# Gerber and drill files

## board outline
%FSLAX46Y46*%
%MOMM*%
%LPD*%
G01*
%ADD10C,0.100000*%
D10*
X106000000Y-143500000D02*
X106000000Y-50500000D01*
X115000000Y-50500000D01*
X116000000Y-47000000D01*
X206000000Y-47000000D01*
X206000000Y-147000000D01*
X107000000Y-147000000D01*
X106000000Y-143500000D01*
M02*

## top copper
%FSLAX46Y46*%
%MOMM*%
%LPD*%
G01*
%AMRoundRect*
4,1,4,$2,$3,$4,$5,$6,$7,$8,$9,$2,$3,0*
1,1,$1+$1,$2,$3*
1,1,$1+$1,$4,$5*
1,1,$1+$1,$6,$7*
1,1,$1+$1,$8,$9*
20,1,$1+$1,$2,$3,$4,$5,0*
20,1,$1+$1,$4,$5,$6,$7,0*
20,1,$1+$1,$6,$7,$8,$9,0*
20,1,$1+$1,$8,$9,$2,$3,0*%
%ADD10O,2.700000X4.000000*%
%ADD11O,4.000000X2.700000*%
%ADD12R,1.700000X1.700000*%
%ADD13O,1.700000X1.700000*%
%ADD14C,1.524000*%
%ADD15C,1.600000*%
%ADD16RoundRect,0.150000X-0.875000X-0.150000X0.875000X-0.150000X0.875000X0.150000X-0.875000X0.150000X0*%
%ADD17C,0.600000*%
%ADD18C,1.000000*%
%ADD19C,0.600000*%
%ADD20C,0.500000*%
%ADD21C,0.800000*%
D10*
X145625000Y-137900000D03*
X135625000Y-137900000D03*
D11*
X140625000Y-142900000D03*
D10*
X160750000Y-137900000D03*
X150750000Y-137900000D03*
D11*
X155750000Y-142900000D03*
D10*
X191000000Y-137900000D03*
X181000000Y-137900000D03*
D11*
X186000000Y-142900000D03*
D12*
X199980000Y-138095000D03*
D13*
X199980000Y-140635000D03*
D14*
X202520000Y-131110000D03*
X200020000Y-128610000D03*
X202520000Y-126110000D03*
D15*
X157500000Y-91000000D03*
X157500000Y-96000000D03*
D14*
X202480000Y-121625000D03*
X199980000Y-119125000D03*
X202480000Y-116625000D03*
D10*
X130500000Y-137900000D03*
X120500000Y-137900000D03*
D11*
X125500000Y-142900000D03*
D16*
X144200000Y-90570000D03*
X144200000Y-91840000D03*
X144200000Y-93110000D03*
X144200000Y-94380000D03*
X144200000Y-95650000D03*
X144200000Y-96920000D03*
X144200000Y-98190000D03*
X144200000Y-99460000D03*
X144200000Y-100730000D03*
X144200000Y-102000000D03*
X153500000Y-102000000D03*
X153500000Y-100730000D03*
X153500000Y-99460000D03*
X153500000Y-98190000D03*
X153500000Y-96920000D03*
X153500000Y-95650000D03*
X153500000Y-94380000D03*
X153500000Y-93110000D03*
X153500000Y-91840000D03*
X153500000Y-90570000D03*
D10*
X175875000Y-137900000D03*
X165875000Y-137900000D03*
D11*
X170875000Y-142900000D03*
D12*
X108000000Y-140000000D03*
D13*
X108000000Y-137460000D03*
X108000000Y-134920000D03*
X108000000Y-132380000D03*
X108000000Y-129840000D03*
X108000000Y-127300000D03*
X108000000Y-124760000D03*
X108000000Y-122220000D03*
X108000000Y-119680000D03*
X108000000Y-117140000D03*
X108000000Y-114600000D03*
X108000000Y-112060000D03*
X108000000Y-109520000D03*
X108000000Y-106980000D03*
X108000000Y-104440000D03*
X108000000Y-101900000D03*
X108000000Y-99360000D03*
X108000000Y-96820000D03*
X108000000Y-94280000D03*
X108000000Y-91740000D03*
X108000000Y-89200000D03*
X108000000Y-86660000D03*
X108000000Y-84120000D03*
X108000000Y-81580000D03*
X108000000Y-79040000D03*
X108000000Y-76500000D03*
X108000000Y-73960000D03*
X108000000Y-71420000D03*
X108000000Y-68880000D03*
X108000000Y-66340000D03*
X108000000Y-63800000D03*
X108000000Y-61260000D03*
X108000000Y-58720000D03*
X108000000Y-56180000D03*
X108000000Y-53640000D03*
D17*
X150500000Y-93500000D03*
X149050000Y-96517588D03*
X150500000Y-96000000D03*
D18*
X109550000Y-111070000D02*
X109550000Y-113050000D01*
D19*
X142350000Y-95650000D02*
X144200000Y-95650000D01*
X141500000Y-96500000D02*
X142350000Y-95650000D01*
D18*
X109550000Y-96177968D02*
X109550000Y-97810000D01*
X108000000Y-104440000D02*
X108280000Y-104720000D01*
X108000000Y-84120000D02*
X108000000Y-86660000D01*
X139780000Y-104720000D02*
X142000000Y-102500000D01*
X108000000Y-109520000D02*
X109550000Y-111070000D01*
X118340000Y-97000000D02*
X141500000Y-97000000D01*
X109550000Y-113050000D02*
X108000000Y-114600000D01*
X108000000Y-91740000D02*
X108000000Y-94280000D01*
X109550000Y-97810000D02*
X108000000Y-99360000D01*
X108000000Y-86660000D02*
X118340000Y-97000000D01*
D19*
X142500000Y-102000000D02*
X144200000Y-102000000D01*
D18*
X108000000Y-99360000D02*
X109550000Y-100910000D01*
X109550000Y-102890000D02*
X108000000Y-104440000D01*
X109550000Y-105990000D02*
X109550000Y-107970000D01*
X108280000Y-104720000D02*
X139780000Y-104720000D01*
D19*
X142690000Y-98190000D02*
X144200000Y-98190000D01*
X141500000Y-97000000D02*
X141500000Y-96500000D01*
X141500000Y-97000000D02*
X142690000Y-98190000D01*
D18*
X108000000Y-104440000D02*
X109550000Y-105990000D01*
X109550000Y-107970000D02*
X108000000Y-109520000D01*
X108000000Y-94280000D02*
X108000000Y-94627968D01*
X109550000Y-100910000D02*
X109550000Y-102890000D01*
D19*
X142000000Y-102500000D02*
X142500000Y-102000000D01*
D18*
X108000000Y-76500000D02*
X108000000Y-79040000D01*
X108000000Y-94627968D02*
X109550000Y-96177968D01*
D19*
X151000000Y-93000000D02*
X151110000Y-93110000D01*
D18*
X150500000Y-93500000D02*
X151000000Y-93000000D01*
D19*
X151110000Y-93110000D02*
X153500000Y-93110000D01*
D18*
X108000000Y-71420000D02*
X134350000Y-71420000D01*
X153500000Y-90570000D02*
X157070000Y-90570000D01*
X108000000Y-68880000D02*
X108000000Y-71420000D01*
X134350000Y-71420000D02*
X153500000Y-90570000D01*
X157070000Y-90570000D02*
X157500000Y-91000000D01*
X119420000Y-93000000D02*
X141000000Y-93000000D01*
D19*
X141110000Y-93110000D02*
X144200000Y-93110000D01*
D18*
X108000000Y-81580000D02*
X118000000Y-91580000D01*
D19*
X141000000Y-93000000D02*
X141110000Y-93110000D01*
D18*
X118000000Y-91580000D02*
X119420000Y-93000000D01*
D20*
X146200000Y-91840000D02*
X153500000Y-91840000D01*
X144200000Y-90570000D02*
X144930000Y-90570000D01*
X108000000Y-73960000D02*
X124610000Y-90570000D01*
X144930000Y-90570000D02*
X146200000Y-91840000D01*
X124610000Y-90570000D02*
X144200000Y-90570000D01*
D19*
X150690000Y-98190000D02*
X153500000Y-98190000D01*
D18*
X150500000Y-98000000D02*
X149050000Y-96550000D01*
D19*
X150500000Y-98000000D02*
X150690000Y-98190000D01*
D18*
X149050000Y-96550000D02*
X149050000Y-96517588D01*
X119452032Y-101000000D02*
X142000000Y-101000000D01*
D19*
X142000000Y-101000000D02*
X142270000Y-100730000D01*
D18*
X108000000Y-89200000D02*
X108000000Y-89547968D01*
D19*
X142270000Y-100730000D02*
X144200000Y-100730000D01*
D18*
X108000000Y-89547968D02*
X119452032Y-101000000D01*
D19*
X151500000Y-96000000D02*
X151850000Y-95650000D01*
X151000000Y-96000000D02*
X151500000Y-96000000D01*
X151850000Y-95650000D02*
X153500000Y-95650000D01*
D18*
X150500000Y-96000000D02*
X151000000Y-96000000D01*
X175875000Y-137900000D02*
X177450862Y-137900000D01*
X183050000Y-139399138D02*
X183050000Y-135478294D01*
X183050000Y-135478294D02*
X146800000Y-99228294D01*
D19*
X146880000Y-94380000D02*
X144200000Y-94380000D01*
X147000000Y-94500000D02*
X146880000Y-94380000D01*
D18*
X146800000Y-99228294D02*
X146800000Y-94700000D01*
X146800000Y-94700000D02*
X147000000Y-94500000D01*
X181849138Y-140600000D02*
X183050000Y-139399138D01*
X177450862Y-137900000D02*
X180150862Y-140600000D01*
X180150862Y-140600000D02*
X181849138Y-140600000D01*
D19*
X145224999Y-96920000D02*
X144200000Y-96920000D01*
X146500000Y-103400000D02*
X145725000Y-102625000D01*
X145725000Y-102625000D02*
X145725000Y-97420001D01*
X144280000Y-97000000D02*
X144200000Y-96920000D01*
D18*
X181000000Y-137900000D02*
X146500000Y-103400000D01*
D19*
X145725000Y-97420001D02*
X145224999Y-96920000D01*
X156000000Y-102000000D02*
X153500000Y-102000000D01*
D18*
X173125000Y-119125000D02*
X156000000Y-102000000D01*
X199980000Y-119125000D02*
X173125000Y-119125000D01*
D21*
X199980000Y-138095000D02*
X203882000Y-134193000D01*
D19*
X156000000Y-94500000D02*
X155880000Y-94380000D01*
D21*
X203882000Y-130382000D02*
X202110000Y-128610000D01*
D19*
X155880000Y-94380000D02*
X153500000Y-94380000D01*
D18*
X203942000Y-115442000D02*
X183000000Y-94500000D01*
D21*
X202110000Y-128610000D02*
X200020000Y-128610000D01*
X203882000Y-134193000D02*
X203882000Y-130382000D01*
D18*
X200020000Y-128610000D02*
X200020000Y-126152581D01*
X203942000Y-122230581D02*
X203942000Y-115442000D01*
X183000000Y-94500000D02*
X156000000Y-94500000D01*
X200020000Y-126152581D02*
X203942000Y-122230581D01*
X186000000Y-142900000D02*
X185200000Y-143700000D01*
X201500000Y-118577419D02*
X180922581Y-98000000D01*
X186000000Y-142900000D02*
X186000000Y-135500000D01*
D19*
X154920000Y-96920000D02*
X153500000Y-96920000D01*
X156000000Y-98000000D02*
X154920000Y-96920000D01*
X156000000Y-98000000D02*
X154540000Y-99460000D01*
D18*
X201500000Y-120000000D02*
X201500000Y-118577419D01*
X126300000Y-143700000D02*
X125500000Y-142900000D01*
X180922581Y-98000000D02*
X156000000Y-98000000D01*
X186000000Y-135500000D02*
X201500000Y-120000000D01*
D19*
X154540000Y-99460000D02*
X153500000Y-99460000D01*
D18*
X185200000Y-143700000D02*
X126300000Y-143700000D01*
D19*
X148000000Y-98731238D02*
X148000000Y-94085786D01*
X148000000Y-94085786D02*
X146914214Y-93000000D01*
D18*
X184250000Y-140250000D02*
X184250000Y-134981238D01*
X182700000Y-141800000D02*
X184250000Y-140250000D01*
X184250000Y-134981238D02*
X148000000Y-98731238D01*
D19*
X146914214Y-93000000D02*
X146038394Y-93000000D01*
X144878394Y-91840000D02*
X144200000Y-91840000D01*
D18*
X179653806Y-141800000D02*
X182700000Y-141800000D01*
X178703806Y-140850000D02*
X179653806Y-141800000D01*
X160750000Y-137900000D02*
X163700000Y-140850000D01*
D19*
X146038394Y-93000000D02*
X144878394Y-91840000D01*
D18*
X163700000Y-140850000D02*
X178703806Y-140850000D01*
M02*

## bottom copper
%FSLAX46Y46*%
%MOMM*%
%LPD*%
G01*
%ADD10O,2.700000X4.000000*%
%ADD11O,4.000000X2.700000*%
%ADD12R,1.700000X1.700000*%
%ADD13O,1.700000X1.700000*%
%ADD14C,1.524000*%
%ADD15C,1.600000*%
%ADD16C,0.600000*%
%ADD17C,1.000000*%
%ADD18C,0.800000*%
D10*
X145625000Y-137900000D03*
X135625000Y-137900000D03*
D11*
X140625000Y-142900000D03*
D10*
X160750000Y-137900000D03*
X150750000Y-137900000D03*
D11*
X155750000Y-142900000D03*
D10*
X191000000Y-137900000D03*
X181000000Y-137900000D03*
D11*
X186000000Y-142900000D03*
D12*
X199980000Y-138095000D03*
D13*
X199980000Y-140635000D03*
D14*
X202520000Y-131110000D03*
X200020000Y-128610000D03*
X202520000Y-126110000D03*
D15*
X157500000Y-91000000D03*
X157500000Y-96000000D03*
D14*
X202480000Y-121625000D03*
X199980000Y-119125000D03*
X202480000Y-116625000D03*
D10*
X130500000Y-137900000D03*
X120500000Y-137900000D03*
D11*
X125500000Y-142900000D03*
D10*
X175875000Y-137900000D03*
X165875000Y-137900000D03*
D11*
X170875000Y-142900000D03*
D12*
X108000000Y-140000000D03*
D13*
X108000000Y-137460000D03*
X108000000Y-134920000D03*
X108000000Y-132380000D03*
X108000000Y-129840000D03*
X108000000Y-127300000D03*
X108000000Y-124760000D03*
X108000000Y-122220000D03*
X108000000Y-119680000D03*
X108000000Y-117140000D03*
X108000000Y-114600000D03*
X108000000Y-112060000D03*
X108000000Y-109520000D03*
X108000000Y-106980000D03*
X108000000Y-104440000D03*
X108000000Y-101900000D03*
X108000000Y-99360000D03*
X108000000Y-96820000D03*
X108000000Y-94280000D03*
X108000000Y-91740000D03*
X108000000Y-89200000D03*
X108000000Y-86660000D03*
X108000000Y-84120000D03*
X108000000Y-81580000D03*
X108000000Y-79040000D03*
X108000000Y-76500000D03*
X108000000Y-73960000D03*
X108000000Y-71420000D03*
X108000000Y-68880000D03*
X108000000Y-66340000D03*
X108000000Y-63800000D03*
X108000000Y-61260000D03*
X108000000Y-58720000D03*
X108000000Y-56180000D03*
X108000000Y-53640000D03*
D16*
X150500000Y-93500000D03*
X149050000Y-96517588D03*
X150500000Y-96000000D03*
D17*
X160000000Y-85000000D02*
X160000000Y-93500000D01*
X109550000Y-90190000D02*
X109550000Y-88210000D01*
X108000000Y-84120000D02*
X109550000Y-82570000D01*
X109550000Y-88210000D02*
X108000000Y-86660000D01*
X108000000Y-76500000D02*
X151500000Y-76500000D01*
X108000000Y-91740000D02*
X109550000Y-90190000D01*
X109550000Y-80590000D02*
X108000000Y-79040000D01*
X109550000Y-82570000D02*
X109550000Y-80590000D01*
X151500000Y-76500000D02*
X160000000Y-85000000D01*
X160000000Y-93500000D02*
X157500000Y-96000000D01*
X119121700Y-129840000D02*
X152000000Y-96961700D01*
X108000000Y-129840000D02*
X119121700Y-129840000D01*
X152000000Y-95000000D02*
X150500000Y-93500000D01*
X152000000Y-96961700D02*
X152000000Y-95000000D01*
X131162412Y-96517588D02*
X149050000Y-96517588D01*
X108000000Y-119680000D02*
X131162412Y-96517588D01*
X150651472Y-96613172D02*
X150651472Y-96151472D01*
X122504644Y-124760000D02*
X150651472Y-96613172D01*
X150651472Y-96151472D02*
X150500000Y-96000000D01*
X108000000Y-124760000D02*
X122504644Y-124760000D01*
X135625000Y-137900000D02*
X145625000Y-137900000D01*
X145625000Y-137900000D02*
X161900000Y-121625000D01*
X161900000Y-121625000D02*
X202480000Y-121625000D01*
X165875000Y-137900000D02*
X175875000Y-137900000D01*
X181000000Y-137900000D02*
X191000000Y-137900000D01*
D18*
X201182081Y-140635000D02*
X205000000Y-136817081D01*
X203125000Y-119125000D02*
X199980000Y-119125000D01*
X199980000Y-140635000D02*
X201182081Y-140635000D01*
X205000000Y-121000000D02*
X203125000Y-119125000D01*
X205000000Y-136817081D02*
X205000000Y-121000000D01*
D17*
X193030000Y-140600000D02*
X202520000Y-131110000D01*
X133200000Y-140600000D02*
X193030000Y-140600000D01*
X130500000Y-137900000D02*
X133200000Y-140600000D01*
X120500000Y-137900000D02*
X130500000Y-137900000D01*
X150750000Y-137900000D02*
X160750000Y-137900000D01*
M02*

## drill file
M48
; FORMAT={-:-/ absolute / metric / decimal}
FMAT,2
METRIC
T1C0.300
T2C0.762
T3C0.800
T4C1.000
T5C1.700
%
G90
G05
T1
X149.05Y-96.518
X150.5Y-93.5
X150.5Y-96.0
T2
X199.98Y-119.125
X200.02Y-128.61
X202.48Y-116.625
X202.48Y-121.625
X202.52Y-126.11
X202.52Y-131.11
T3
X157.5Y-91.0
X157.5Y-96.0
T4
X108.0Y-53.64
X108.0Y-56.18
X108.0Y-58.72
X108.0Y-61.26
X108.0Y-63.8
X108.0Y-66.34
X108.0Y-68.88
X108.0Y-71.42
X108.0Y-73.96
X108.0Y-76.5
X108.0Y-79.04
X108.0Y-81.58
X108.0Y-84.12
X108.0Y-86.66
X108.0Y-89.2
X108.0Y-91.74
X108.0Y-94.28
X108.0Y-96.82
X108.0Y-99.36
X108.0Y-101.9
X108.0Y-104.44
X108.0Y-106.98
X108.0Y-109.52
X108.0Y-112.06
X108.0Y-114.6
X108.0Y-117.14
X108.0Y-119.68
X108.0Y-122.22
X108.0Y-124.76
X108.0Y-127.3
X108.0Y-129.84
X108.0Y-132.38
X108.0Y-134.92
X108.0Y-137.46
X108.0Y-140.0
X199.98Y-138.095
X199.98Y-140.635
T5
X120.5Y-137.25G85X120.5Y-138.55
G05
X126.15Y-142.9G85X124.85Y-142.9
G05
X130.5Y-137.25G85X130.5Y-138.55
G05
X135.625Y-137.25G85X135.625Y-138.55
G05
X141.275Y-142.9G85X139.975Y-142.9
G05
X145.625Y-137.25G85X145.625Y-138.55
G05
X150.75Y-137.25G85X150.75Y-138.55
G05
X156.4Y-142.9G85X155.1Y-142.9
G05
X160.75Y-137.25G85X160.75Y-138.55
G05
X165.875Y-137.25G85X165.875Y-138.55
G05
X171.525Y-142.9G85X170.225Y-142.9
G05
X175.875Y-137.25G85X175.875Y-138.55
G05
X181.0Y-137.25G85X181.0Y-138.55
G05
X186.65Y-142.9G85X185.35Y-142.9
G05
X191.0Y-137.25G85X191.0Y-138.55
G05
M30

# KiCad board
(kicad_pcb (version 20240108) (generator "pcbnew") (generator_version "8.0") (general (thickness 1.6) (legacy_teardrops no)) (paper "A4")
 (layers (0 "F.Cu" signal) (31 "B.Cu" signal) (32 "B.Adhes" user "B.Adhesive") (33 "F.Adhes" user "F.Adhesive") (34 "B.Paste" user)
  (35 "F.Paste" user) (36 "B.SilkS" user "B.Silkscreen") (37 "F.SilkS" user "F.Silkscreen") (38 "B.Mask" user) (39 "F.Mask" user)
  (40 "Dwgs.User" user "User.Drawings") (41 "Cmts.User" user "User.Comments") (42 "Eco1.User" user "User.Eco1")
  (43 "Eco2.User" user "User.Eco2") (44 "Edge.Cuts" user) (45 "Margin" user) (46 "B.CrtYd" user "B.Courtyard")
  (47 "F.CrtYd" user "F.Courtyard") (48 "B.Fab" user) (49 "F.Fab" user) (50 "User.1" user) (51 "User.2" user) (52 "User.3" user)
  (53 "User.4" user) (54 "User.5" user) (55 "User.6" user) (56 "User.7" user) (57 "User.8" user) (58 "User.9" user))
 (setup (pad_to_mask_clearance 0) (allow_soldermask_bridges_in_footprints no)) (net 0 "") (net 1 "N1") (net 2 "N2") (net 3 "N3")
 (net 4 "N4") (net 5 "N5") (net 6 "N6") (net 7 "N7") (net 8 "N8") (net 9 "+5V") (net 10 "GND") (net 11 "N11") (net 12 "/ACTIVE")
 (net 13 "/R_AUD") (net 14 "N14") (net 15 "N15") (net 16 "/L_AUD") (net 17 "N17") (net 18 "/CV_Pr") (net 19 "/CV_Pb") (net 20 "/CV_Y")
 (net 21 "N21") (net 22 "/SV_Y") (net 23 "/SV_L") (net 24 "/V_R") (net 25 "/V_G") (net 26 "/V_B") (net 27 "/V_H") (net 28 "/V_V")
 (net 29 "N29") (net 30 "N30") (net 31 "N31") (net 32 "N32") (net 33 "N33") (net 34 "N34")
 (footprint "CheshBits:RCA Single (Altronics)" (layer "F.Cu") (at 140.625 137.9 180)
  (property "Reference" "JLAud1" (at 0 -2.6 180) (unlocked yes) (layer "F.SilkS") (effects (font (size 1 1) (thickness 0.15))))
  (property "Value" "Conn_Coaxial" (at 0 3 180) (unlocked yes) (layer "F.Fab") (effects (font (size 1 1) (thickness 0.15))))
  (pad "1" thru_hole oval (at -5 0 270) (size 4 2.7) (drill oval 3 1.7) (layers "*.Cu" "*.Mask") (remove_unused_layers no) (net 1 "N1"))
  (pad "1" thru_hole oval (at 5 0 270) (size 4 2.7) (drill oval 3 1.7) (layers "*.Cu" "*.Mask") (remove_unused_layers no) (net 1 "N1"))
  (pad "2" thru_hole oval (at 0 -5 180) (size 4 2.7) (drill oval 3 1.7) (layers "*.Cu" "*.Mask") (remove_unused_layers no) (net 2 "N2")))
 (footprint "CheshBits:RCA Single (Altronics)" (layer "F.Cu") (at 155.75 137.9 180)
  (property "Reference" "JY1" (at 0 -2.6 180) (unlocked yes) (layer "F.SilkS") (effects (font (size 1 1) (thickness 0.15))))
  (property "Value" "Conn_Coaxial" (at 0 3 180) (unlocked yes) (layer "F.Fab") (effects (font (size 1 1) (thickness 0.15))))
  (pad "1" thru_hole oval (at -5 0 270) (size 4 2.7) (drill oval 3 1.7) (layers "*.Cu" "*.Mask") (remove_unused_layers no) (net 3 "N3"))
  (pad "1" thru_hole oval (at 5 0 270) (size 4 2.7) (drill oval 3 1.7) (layers "*.Cu" "*.Mask") (remove_unused_layers no) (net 3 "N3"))
  (pad "2" thru_hole oval (at 0 -5 180) (size 4 2.7) (drill oval 3 1.7) (layers "*.Cu" "*.Mask") (remove_unused_layers no) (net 2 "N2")))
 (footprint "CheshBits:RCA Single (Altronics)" (layer "F.Cu") (at 186 137.9 180)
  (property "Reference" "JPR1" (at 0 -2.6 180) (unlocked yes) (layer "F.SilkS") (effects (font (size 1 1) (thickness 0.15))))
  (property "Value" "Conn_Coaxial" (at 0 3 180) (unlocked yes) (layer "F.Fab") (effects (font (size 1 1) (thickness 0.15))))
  (pad "1" thru_hole oval (at -5 0 270) (size 4 2.7) (drill oval 3 1.7) (layers "*.Cu" "*.Mask") (remove_unused_layers no) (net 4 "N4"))
  (pad "1" thru_hole oval (at 5 0 270) (size 4 2.7) (drill oval 3 1.7) (layers "*.Cu" "*.Mask") (remove_unused_layers no) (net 4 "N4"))
  (pad "2" thru_hole oval (at 0 -5 180) (size 4 2.7) (drill oval 3 1.7) (layers "*.Cu" "*.Mask") (remove_unused_layers no) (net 2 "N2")))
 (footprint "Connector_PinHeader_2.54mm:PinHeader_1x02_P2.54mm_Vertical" (layer "F.Cu") (at 199.98 138.095)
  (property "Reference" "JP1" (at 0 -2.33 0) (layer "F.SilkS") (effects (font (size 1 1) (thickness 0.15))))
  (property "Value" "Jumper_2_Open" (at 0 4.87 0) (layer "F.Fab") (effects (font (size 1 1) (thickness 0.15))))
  (pad "1" thru_hole rect (at 0 0) (size 1.7 1.7) (drill 1) (layers "*.Cu" "*.Mask") (remove_unused_layers no) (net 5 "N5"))
  (pad "2" thru_hole oval (at 0 2.54) (size 1.7 1.7) (drill 1) (layers "*.Cu" "*.Mask") (remove_unused_layers no) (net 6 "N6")))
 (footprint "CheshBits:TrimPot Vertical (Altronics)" (layer "F.Cu") (at 193.62 128.61 90)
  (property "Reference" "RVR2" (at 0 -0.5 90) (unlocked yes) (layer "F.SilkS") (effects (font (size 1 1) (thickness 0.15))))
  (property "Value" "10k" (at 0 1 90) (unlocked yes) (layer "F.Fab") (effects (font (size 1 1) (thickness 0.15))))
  (pad "1" thru_hole circle (at -2.5 8.9 90) (size 1.524 1.524) (drill 0.762) (layers "*.Cu" "*.Mask") (remove_unused_layers no)
   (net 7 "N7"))
  (pad "2" thru_hole circle (at 0 6.4 90) (size 1.524 1.524) (drill 0.762) (layers "*.Cu" "*.Mask") (remove_unused_layers no) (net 5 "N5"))
  (pad "3" thru_hole circle (at 2.5 8.9 90) (size 1.524 1.524) (drill 0.762) (layers "*.Cu" "*.Mask") (remove_unused_layers no) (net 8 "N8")))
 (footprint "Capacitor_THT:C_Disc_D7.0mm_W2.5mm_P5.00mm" (layer "F.Cu") (at 157.5 91 -90)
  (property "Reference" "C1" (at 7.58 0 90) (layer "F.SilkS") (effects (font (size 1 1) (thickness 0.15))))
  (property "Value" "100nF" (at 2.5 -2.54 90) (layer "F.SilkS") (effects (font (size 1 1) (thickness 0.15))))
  (pad "1" thru_hole circle (at 0 0 270) (size 1.6 1.6) (drill 0.8) (layers "*.Cu" "*.Mask") (remove_unused_layers no) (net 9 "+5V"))
  (pad "2" thru_hole circle (at 5 0 270) (size 1.6 1.6) (drill 0.8) (layers "*.Cu" "*.Mask") (remove_unused_layers no) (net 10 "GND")))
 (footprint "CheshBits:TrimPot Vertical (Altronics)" (layer "F.Cu") (at 193.58 119.125 90)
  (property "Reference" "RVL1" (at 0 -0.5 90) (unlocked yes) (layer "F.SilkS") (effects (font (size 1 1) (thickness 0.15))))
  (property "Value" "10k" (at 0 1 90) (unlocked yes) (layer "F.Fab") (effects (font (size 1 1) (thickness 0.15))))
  (pad "1" thru_hole circle (at -2.5 8.9 90) (size 1.524 1.524) (drill 0.762) (layers "*.Cu" "*.Mask") (remove_unused_layers no)
   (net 1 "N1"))
  (pad "2" thru_hole circle (at 0 6.4 90) (size 1.524 1.524) (drill 0.762) (layers "*.Cu" "*.Mask") (remove_unused_layers no) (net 6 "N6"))
  (pad "3" thru_hole circle (at 2.5 8.9 90) (size 1.524 1.524) (drill 0.762) (layers "*.Cu" "*.Mask") (remove_unused_layers no)
   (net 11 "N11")))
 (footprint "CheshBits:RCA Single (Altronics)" (layer "F.Cu") (at 125.5 137.9 180)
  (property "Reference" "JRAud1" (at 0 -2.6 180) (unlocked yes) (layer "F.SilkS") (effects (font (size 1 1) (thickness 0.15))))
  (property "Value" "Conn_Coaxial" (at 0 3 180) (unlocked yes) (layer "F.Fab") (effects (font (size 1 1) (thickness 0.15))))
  (pad "1" thru_hole oval (at -5 0 270) (size 4 2.7) (drill oval 3 1.7) (layers "*.Cu" "*.Mask") (remove_unused_layers no) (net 7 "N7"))
  (pad "1" thru_hole oval (at 5 0 270) (size 4 2.7) (drill oval 3 1.7) (layers "*.Cu" "*.Mask") (remove_unused_layers no) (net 7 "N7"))
  (pad "2" thru_hole oval (at 0 -5 180) (size 4 2.7) (drill oval 3 1.7) (layers "*.Cu" "*.Mask") (remove_unused_layers no) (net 2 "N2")))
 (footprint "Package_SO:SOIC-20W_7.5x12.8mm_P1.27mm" (layer "F.Cu") (at 148.85 96.285)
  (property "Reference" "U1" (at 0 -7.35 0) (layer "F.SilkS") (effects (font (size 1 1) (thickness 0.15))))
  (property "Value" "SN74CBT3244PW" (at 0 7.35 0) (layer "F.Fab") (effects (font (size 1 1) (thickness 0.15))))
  (pad "1" smd roundrect (at -4.65 -5.715) (size 2.05 0.6) (layers "F.Cu" "F.Paste" "F.Mask") (roundrect_rratio 0.25) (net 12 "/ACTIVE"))
  (pad "2" smd roundrect (at -4.65 -4.445) (size 2.05 0.6) (layers "F.Cu" "F.Paste" "F.Mask") (roundrect_rratio 0.25) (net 3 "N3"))
  (pad "3" smd roundrect (at -4.65 -3.175) (size 2.05 0.6) (layers "F.Cu" "F.Paste" "F.Mask") (roundrect_rratio 0.25) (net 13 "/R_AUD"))
  (pad "4" smd roundrect (at -4.65 -1.905) (size 2.05 0.6) (layers "F.Cu" "F.Paste" "F.Mask") (roundrect_rratio 0.25) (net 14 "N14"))
  (pad "5" smd roundrect (at -4.65 -0.635) (size 2.05 0.6) (layers "F.Cu" "F.Paste" "F.Mask") (roundrect_rratio 0.25) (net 10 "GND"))
  (pad "6" smd roundrect (at -4.65 0.635) (size 2.05 0.6) (layers "F.Cu" "F.Paste" "F.Mask") (roundrect_rratio 0.25) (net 4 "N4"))
  (pad "7" smd roundrect (at -4.65 1.905) (size 2.05 0.6) (layers "F.Cu" "F.Paste" "F.Mask") (roundrect_rratio 0.25) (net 10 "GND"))
  (pad "8" smd roundrect (at -4.65 3.175) (size 2.05 0.6) (layers "F.Cu" "F.Paste" "F.Mask") (roundrect_rratio 0.25) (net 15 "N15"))
  (pad "9" smd roundrect (at -4.65 4.445) (size 2.05 0.6) (layers "F.Cu" "F.Paste" "F.Mask") (roundrect_rratio 0.25) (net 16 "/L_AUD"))
  (pad "10" smd roundrect (at -4.65 5.715) (size 2.05 0.6) (layers "F.Cu" "F.Paste" "F.Mask") (roundrect_rratio 0.25) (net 10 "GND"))
  (pad "11" smd roundrect (at 4.65 5.715) (size 2.05 0.6) (layers "F.Cu" "F.Paste" "F.Mask") (roundrect_rratio 0.25) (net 6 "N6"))
  (pad "12" smd roundrect (at 4.65 4.445) (size 2.05 0.6) (layers "F.Cu" "F.Paste" "F.Mask") (roundrect_rratio 0.25) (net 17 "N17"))
  (pad "13" smd roundrect (at 4.65 3.175) (size 2.05 0.6) (layers "F.Cu" "F.Paste" "F.Mask") (roundrect_rratio 0.25) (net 2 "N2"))
  (pad "14" smd roundrect (at 4.65 1.905) (size 2.05 0.6) (layers "F.Cu" "F.Paste" "F.Mask") (roundrect_rratio 0.25) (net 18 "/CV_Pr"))
  (pad "15" smd roundrect (at 4.65 0.635) (size 2.05 0.6) (layers "F.Cu" "F.Paste" "F.Mask") (roundrect_rratio 0.25) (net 2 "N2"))
  (pad "16" smd roundrect (at 4.65 -0.635) (size 2.05 0.6) (layers "F.Cu" "F.Paste" "F.Mask") (roundrect_rratio 0.25) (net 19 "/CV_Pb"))
  (pad "17" smd roundrect (at 4.65 -1.905) (size 2.05 0.6) (layers "F.Cu" "F.Paste" "F.Mask") (roundrect_rratio 0.25) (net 5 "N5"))
  (pad "18" smd roundrect (at 4.65 -3.175) (size 2.05 0.6) (layers "F.Cu" "F.Paste" "F.Mask") (roundrect_rratio 0.25) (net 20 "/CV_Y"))
  (pad "19" smd roundrect (at 4.65 -4.445) (size 2.05 0.6) (layers "F.Cu" "F.Paste" "F.Mask") (roundrect_rratio 0.25) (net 12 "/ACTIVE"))
  (pad "20" smd roundrect (at 4.65 -5.715) (size 2.05 0.6) (layers "F.Cu" "F.Paste" "F.Mask") (roundrect_rratio 0.25) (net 9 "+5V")))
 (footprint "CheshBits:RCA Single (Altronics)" (layer "F.Cu") (at 170.875 137.9 180)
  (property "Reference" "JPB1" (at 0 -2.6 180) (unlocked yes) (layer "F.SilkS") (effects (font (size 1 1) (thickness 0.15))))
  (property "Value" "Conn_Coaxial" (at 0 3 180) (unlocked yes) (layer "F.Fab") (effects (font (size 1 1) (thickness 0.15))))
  (pad "1" thru_hole oval (at -5 0 270) (size 4 2.7) (drill oval 3 1.7) (layers "*.Cu" "*.Mask") (remove_unused_layers no) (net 14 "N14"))
  (pad "1" thru_hole oval (at 5 0 270) (size 4 2.7) (drill oval 3 1.7) (layers "*.Cu" "*.Mask") (remove_unused_layers no) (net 14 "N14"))
  (pad "2" thru_hole oval (at 0 -5 180) (size 4 2.7) (drill oval 3 1.7) (layers "*.Cu" "*.Mask") (remove_unused_layers no) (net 2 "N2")))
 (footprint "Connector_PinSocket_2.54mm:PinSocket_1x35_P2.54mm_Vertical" (layer "B.Cu") (at 108 140)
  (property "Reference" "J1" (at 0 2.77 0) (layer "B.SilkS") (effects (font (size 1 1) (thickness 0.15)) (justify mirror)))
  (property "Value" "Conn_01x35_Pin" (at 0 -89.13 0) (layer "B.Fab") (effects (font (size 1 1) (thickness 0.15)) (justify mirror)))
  (pad "1" thru_hole rect (at 0 0) (size 1.7 1.7) (drill 1) (layers "*.Cu" "*.Mask") (remove_unused_layers no) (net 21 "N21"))
  (pad "2" thru_hole oval (at 0 -2.54) (size 1.7 1.7) (drill 1) (layers "*.Cu" "*.Mask") (remove_unused_layers no) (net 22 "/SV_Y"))
  (pad "3" thru_hole oval (at 0 -5.08) (size 1.7 1.7) (drill 1) (layers "*.Cu" "*.Mask") (remove_unused_layers no) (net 10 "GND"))
  (pad "4" thru_hole oval (at 0 -7.62) (size 1.7 1.7) (drill 1) (layers "*.Cu" "*.Mask") (remove_unused_layers no) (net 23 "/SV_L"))
  (pad "5" thru_hole oval (at 0 -10.16) (size 1.7 1.7) (drill 1) (layers "*.Cu" "*.Mask") (remove_unused_layers no) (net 20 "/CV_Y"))
  (pad "6" thru_hole oval (at 0 -12.7) (size 1.7 1.7) (drill 1) (layers "*.Cu" "*.Mask") (remove_unused_layers no) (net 10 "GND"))
  (pad "7" thru_hole oval (at 0 -15.24) (size 1.7 1.7) (drill 1) (layers "*.Cu" "*.Mask") (remove_unused_layers no) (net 19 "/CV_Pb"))
  (pad "8" thru_hole oval (at 0 -17.78) (size 1.7 1.7) (drill 1) (layers "*.Cu" "*.Mask") (remove_unused_layers no) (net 10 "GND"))
  (pad "9" thru_hole oval (at 0 -20.32) (size 1.7 1.7) (drill 1) (layers "*.Cu" "*.Mask") (remove_unused_layers no) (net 18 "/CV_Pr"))
  (pad "10" thru_hole oval (at 0 -22.86) (size 1.7 1.7) (drill 1) (layers "*.Cu" "*.Mask") (remove_unused_layers no) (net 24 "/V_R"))
  (pad "11" thru_hole oval (at 0 -25.4) (size 1.7 1.7) (drill 1) (layers "*.Cu" "*.Mask") (remove_unused_layers no) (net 10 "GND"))
  (pad "12" thru_hole oval (at 0 -27.94) (size 1.7 1.7) (drill 1) (layers "*.Cu" "*.Mask") (remove_unused_layers no) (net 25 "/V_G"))
  (pad "13" thru_hole oval (at 0 -30.48) (size 1.7 1.7) (drill 1) (layers "*.Cu" "*.Mask") (remove_unused_layers no) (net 10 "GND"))
  (pad "14" thru_hole oval (at 0 -33.02) (size 1.7 1.7) (drill 1) (layers "*.Cu" "*.Mask") (remove_unused_layers no) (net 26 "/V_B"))
  (pad "15" thru_hole oval (at 0 -35.56) (size 1.7 1.7) (drill 1) (layers "*.Cu" "*.Mask") (remove_unused_layers no) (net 10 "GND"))
  (pad "16" thru_hole oval (at 0 -38.1) (size 1.7 1.7) (drill 1) (layers "*.Cu" "*.Mask") (remove_unused_layers no) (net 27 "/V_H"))
  (pad "17" thru_hole oval (at 0 -40.64) (size 1.7 1.7) (drill 1) (layers "*.Cu" "*.Mask") (remove_unused_layers no) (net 10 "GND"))
  (pad "18" thru_hole oval (at 0 -43.18) (size 1.7 1.7) (drill 1) (layers "*.Cu" "*.Mask") (remove_unused_layers no) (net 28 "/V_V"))
  (pad "19" thru_hole oval (at 0 -45.72) (size 1.7 1.7) (drill 1) (layers "*.Cu" "*.Mask") (remove_unused_layers no) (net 10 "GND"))
  (pad "20" thru_hole oval (at 0 -48.26) (size 1.7 1.7) (drill 1) (layers "*.Cu" "*.Mask") (remove_unused_layers no) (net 10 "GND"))
  (pad "21" thru_hole oval (at 0 -50.8) (size 1.7 1.7) (drill 1) (layers "*.Cu" "*.Mask") (remove_unused_layers no) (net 16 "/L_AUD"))
  (pad "22" thru_hole oval (at 0 -53.34) (size 1.7 1.7) (drill 1) (layers "*.Cu" "*.Mask") (remove_unused_layers no) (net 10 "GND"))
  (pad "23" thru_hole oval (at 0 -55.88) (size 1.7 1.7) (drill 1) (layers "*.Cu" "*.Mask") (remove_unused_layers no) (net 10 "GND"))
  (pad "24" thru_hole oval (at 0 -58.42) (size 1.7 1.7) (drill 1) (layers "*.Cu" "*.Mask") (remove_unused_layers no) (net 13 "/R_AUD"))
  (pad "25" thru_hole oval (at 0 -60.96) (size 1.7 1.7) (drill 1) (layers "*.Cu" "*.Mask") (remove_unused_layers no) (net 10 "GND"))
  (pad "26" thru_hole oval (at 0 -63.5) (size 1.7 1.7) (drill 1) (layers "*.Cu" "*.Mask") (remove_unused_layers no) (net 10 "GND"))
  (pad "27" thru_hole oval (at 0 -66.04) (size 1.7 1.7) (drill 1) (layers "*.Cu" "*.Mask") (remove_unused_layers no) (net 12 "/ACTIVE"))
  (pad "28" thru_hole oval (at 0 -68.58) (size 1.7 1.7) (drill 1) (layers "*.Cu" "*.Mask") (remove_unused_layers no) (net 9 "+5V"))
  (pad "29" thru_hole oval (at 0 -71.12) (size 1.7 1.7) (drill 1) (layers "*.Cu" "*.Mask") (remove_unused_layers no) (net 9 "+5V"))
  (pad "30" thru_hole oval (at 0 -73.66) (size 1.7 1.7) (drill 1) (layers "*.Cu" "*.Mask") (remove_unused_layers no) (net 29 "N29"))
  (pad "31" thru_hole oval (at 0 -76.2) (size 1.7 1.7) (drill 1) (layers "*.Cu" "*.Mask") (remove_unused_layers no) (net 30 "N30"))
  (pad "32" thru_hole oval (at 0 -78.74) (size 1.7 1.7) (drill 1) (layers "*.Cu" "*.Mask") (remove_unused_layers no) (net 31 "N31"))
  (pad "33" thru_hole oval (at 0 -81.28) (size 1.7 1.7) (drill 1) (layers "*.Cu" "*.Mask") (remove_unused_layers no) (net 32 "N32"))
  (pad "34" thru_hole oval (at 0 -83.82) (size 1.7 1.7) (drill 1) (layers "*.Cu" "*.Mask") (remove_unused_layers no) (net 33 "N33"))
  (pad "35" thru_hole oval (at 0 -86.36) (size 1.7 1.7) (drill 1) (layers "*.Cu" "*.Mask") (remove_unused_layers no) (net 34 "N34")))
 (gr_poly
  (pts (xy 106 143.5) (xy 106 50.5) (xy 115 50.5) (xy 116 47) (xy 206 47) (xy 206 147) (xy 107 147)) (stroke (width 0.1) (type solid))
  (fill none) (layer "Edge.Cuts"))
 (segment (start 109.55 111.07) (end 109.55 113.05) (width 1) (layer "F.Cu") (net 10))
 (segment (start 142.35 95.65) (end 144.2 95.65) (width 0.6) (layer "F.Cu") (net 10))
 (segment (start 141.5 96.5) (end 142.35 95.65) (width 0.6) (layer "F.Cu") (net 10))
 (segment (start 109.55 96.177968) (end 109.55 97.81) (width 1) (layer "F.Cu") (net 10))
 (segment (start 108 104.44) (end 108.28 104.72) (width 1) (layer "F.Cu") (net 10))
 (segment (start 108 84.12) (end 108 86.66) (width 1) (layer "F.Cu") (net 10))
 (segment (start 139.78 104.72) (end 142 102.5) (width 1) (layer "F.Cu") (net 10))
 (segment (start 108 109.52) (end 109.55 111.07) (width 1) (layer "F.Cu") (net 10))
 (segment (start 118.34 97) (end 141.5 97) (width 1) (layer "F.Cu") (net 10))
 (segment (start 109.55 113.05) (end 108 114.6) (width 1) (layer "F.Cu") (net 10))
 (segment (start 108 91.74) (end 108 94.28) (width 1) (layer "F.Cu") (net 10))
 (segment (start 109.55 97.81) (end 108 99.36) (width 1) (layer "F.Cu") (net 10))
 (segment (start 108 86.66) (end 118.34 97) (width 1) (layer "F.Cu") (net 10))
 (segment (start 142.5 102) (end 144.2 102) (width 0.6) (layer "F.Cu") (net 10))
 (segment (start 108 99.36) (end 109.55 100.91) (width 1) (layer "F.Cu") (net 10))
 (segment (start 109.55 102.89) (end 108 104.44) (width 1) (layer "F.Cu") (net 10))
 (segment (start 109.55 105.99) (end 109.55 107.97) (width 1) (layer "F.Cu") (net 10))
 (segment (start 108.28 104.72) (end 139.78 104.72) (width 1) (layer "F.Cu") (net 10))
 (segment (start 142.69 98.19) (end 144.2 98.19) (width 0.6) (layer "F.Cu") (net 10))
 (segment (start 141.5 97) (end 141.5 96.5) (width 0.6) (layer "F.Cu") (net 10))
 (segment (start 141.5 97) (end 142.69 98.19) (width 0.6) (layer "F.Cu") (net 10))
 (segment (start 108 104.44) (end 109.55 105.99) (width 1) (layer "F.Cu") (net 10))
 (segment (start 109.55 107.97) (end 108 109.52) (width 1) (layer "F.Cu") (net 10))
 (segment (start 108 94.28) (end 108 94.627968) (width 1) (layer "F.Cu") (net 10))
 (segment (start 109.55 100.91) (end 109.55 102.89) (width 1) (layer "F.Cu") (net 10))
 (segment (start 142 102.5) (end 142.5 102) (width 0.6) (layer "F.Cu") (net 10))
 (segment (start 108 76.5) (end 108 79.04) (width 1) (layer "F.Cu") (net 10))
 (segment (start 108 94.627968) (end 109.55 96.177968) (width 1) (layer "F.Cu") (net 10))
 (segment (start 160 85) (end 160 93.5) (width 1) (layer "B.Cu") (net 10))
 (segment (start 109.55 90.19) (end 109.55 88.21) (width 1) (layer "B.Cu") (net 10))
 (segment (start 108 84.12) (end 109.55 82.57) (width 1) (layer "B.Cu") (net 10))
 (segment (start 109.55 88.21) (end 108 86.66) (width 1) (layer "B.Cu") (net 10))
 (segment (start 108 76.5) (end 151.5 76.5) (width 1) (layer "B.Cu") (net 10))
 (segment (start 108 91.74) (end 109.55 90.19) (width 1) (layer "B.Cu") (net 10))
 (segment (start 109.55 80.59) (end 108 79.04) (width 1) (layer "B.Cu") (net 10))
 (segment (start 109.55 82.57) (end 109.55 80.59) (width 1) (layer "B.Cu") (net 10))
 (segment (start 151.5 76.5) (end 160 85) (width 1) (layer "B.Cu") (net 10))
 (segment (start 160 93.5) (end 157.5 96) (width 1) (layer "B.Cu") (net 10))
 (segment (start 151 93) (end 151.11 93.11) (width 0.6) (layer "F.Cu") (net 20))
 (segment (start 150.5 93.5) (end 151 93) (width 1) (layer "F.Cu") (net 20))
 (segment (start 151.11 93.11) (end 153.5 93.11) (width 0.6) (layer "F.Cu") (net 20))
 (via (at 150.5 93.5) (size 0.6) (drill 0.3) (layers "F.Cu" "B.Cu") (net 20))
 (segment (start 119.1217 129.84) (end 152 96.9617) (width 1) (layer "B.Cu") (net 20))
 (segment (start 108 129.84) (end 119.1217 129.84) (width 1) (layer "B.Cu") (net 20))
 (segment (start 152 95) (end 150.5 93.5) (width 1) (layer "B.Cu") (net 20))
 (segment (start 152 96.9617) (end 152 95) (width 1) (layer "B.Cu") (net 20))
 (segment (start 108 71.42) (end 134.35 71.42) (width 1) (layer "F.Cu") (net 9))
 (segment (start 153.5 90.57) (end 157.07 90.57) (width 1) (layer "F.Cu") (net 9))
 (segment (start 108 68.88) (end 108 71.42) (width 1) (layer "F.Cu") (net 9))
 (segment (start 134.35 71.42) (end 153.5 90.57) (width 1) (layer "F.Cu") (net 9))
 (segment (start 157.07 90.57) (end 157.5 91) (width 1) (layer "F.Cu") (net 9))
 (segment (start 119.42 93) (end 141 93) (width 1) (layer "F.Cu") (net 13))
 (segment (start 141.11 93.11) (end 144.2 93.11) (width 0.6) (layer "F.Cu") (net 13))
 (segment (start 108 81.58) (end 118 91.58) (width 1) (layer "F.Cu") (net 13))
 (segment (start 141 93) (end 141.11 93.11) (width 0.6) (layer "F.Cu") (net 13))
 (segment (start 118 91.58) (end 119.42 93) (width 1) (layer "F.Cu") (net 13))
 (segment (start 146.2 91.84) (end 153.5 91.84) (width 0.5) (layer "F.Cu") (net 12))
 (segment (start 144.2 90.57) (end 144.93 90.57) (width 0.5) (layer "F.Cu") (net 12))
 (segment (start 108 73.96) (end 124.61 90.57) (width 0.5) (layer "F.Cu") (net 12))
 (segment (start 144.93 90.57) (end 146.2 91.84) (width 0.5) (layer "F.Cu") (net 12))
 (segment (start 124.61 90.57) (end 144.2 90.57) (width 0.5) (layer "F.Cu") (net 12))
 (segment (start 150.69 98.19) (end 153.5 98.19) (width 0.6) (layer "F.Cu") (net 18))
 (segment (start 150.5 98) (end 149.05 96.55) (width 1) (layer "F.Cu") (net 18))
 (segment (start 150.5 98) (end 150.69 98.19) (width 0.6) (layer "F.Cu") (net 18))
 (segment (start 149.05 96.55) (end 149.05 96.517588) (width 1) (layer "F.Cu") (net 18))
 (via (at 149.05 96.517588) (size 0.6) (drill 0.3) (layers "F.Cu" "B.Cu") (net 18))
 (segment (start 131.162412 96.517588) (end 149.05 96.517588) (width 1) (layer "B.Cu") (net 18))
 (segment (start 108 119.68) (end 131.162412 96.517588) (width 1) (layer "B.Cu") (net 18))
 (segment (start 119.452032 101) (end 142 101) (width 1) (layer "F.Cu") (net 16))
 (segment (start 142 101) (end 142.27 100.73) (width 0.6) (layer "F.Cu") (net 16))
 (segment (start 108 89.2) (end 108 89.547968) (width 1) (layer "F.Cu") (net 16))
 (segment (start 142.27 100.73) (end 144.2 100.73) (width 0.6) (layer "F.Cu") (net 16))
 (segment (start 108 89.547968) (end 119.452032 101) (width 1) (layer "F.Cu") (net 16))
 (segment (start 151.5 96) (end 151.85 95.65) (width 0.6) (layer "F.Cu") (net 19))
 (segment (start 151 96) (end 151.5 96) (width 0.6) (layer "F.Cu") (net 19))
 (segment (start 151.85 95.65) (end 153.5 95.65) (width 0.6) (layer "F.Cu") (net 19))
 (segment (start 150.5 96) (end 151 96) (width 1) (layer "F.Cu") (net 19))
 (via (at 150.5 96) (size 0.6) (drill 0.3) (layers "F.Cu" "B.Cu") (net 19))
 (segment (start 150.651472 96.613172) (end 150.651472 96.151472) (width 1) (layer "B.Cu") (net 19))
 (segment (start 122.504644 124.76) (end 150.651472 96.613172) (width 1) (layer "B.Cu") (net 19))
 (segment (start 150.651472 96.151472) (end 150.5 96) (width 1) (layer "B.Cu") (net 19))
 (segment (start 108 124.76) (end 122.504644 124.76) (width 1) (layer "B.Cu") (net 19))
 (segment (start 135.625 137.9) (end 145.625 137.9) (width 1) (layer "B.Cu") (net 1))
 (segment (start 145.625 137.9) (end 161.9 121.625) (width 1) (layer "B.Cu") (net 1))
 (segment (start 161.9 121.625) (end 202.48 121.625) (width 1) (layer "B.Cu") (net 1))
 (segment (start 175.875 137.9) (end 177.450862 137.9) (width 1) (layer "F.Cu") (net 14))
 (segment (start 183.05 139.399138) (end 183.05 135.478294) (width 1) (layer "F.Cu") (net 14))
 (segment (start 183.05 135.478294) (end 146.8 99.228294) (width 1) (layer "F.Cu") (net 14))
 (segment (start 146.88 94.38) (end 144.2 94.38) (width 0.6) (layer "F.Cu") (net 14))
 (segment (start 147 94.5) (end 146.88 94.38) (width 0.6) (layer "F.Cu") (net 14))
 (segment (start 146.8 99.228294) (end 146.8 94.7) (width 1) (layer "F.Cu") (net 14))
 (segment (start 146.8 94.7) (end 147 94.5) (width 1) (layer "F.Cu") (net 14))
 (segment (start 181.849138 140.6) (end 183.05 139.399138) (width 1) (layer "F.Cu") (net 14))
 (segment (start 177.450862 137.9) (end 180.150862 140.6) (width 1) (layer "F.Cu") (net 14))
 (segment (start 180.150862 140.6) (end 181.849138 140.6) (width 1) (layer "F.Cu") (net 14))
 (segment (start 165.875 137.9) (end 175.875 137.9) (width 1) (layer "B.Cu") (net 14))
 (segment (start 145.224999 96.92) (end 144.2 96.92) (width 0.6) (layer "F.Cu") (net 4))
 (segment (start 146.5 103.4) (end 145.725 102.625) (width 0.6) (layer "F.Cu") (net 4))
 (segment (start 145.725 102.625) (end 145.725 97.420001) (width 0.6) (layer "F.Cu") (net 4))
 (segment (start 144.28 97) (end 144.2 96.92) (width 0.6) (layer "F.Cu") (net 4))
 (segment (start 181 137.9) (end 146.5 103.4) (width 1) (layer "F.Cu") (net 4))
 (segment (start 145.725 97.420001) (end 145.224999 96.92) (width 0.6) (layer "F.Cu") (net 4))
 (segment (start 181 137.9) (end 191 137.9) (width 1) (layer "B.Cu") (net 4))
 (segment (start 156 102) (end 153.5 102) (width 0.6) (layer "F.Cu") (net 6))
 (segment (start 173.125 119.125) (end 156 102) (width 1) (layer "F.Cu") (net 6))
 (segment (start 199.98 119.125) (end 173.125 119.125) (width 1) (layer "F.Cu") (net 6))
 (segment (start 201.182081 140.635) (end 205 136.817081) (width 0.8) (layer "B.Cu") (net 6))
 (segment (start 203.125 119.125) (end 199.98 119.125) (width 0.8) (layer "B.Cu") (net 6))
 (segment (start 199.98 140.635) (end 201.182081 140.635) (width 0.8) (layer "B.Cu") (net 6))
 (segment (start 205 121) (end 203.125 119.125) (width 0.8) (layer "B.Cu") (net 6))
 (segment (start 205 136.817081) (end 205 121) (width 0.8) (layer "B.Cu") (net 6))
 (segment (start 199.98 138.095) (end 203.882 134.193) (width 0.8) (layer "F.Cu") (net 5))
 (segment (start 156 94.5) (end 155.88 94.38) (width 0.6) (layer "F.Cu") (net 5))
 (segment (start 203.882 130.382) (end 202.11 128.61) (width 0.8) (layer "F.Cu") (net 5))
 (segment (start 155.88 94.38) (end 153.5 94.38) (width 0.6) (layer "F.Cu") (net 5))
 (segment (start 203.942 115.442) (end 183 94.5) (width 1) (layer "F.Cu") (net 5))
 (segment (start 202.11 128.61) (end 200.02 128.61) (width 0.8) (layer "F.Cu") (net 5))
 (segment (start 203.882 134.193) (end 203.882 130.382) (width 0.8) (layer "F.Cu") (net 5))
 (segment (start 200.02 128.61) (end 200.02 126.152581) (width 1) (layer "F.Cu") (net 5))
 (segment (start 203.942 122.230581) (end 203.942 115.442) (width 1) (layer "F.Cu") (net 5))
 (segment (start 183 94.5) (end 156 94.5) (width 1) (layer "F.Cu") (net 5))
 (segment (start 200.02 126.152581) (end 203.942 122.230581) (width 1) (layer "F.Cu") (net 5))
 (segment (start 186 142.9) (end 185.2 143.7) (width 1) (layer "F.Cu") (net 2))
 (segment (start 201.5 118.577419) (end 180.922581 98) (width 1) (layer "F.Cu") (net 2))
 (segment (start 186 142.9) (end 186 135.5) (width 1) (layer "F.Cu") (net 2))
 (segment (start 154.92 96.92) (end 153.5 96.92) (width 0.6) (layer "F.Cu") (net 2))
 (segment (start 156 98) (end 154.92 96.92) (width 0.6) (layer "F.Cu") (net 2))
 (segment (start 156 98) (end 154.54 99.46) (width 0.6) (layer "F.Cu") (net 2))
 (segment (start 201.5 120) (end 201.5 118.577419) (width 1) (layer "F.Cu") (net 2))
 (segment (start 126.3 143.7) (end 125.5 142.9) (width 1) (layer "F.Cu") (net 2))
 (segment (start 180.922581 98) (end 156 98) (width 1) (layer "F.Cu") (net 2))
 (segment (start 186 135.5) (end 201.5 120) (width 1) (layer "F.Cu") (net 2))
 (segment (start 154.54 99.46) (end 153.5 99.46) (width 0.6) (layer "F.Cu") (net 2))
 (segment (start 185.2 143.7) (end 126.3 143.7) (width 1) (layer "F.Cu") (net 2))
 (segment (start 193.03 140.6) (end 202.52 131.11) (width 1) (layer "B.Cu") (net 7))
 (segment (start 133.2 140.6) (end 193.03 140.6) (width 1) (layer "B.Cu") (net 7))
 (segment (start 130.5 137.9) (end 133.2 140.6) (width 1) (layer "B.Cu") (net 7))
 (segment (start 120.5 137.9) (end 130.5 137.9) (width 1) (layer "B.Cu") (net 7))
 (segment (start 148 98.731238) (end 148 94.085786) (width 0.6) (layer "F.Cu") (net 3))
 (segment (start 148 94.085786) (end 146.914214 93) (width 0.6) (layer "F.Cu") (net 3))
 (segment (start 184.25 140.25) (end 184.25 134.981238) (width 1) (layer "F.Cu") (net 3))
 (segment (start 182.7 141.8) (end 184.25 140.25) (width 1) (layer "F.Cu") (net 3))
 (segment (start 184.25 134.981238) (end 148 98.731238) (width 1) (layer "F.Cu") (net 3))
 (segment (start 146.914214 93) (end 146.038394 93) (width 0.6) (layer "F.Cu") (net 3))
 (segment (start 144.878394 91.84) (end 144.2 91.84) (width 0.6) (layer "F.Cu") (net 3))
 (segment (start 179.653806 141.8) (end 182.7 141.8) (width 1) (layer "F.Cu") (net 3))
 (segment (start 178.703806 140.85) (end 179.653806 141.8) (width 1) (layer "F.Cu") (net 3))
 (segment (start 160.75 137.9) (end 163.7 140.85) (width 1) (layer "F.Cu") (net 3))
 (segment (start 146.038394 93) (end 144.878394 91.84) (width 0.6) (layer "F.Cu") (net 3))
 (segment (start 163.7 140.85) (end 178.703806 140.85) (width 1) (layer "F.Cu") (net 3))
 (segment (start 150.75 137.9) (end 160.75 137.9) (width 1) (layer "B.Cu") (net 3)))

